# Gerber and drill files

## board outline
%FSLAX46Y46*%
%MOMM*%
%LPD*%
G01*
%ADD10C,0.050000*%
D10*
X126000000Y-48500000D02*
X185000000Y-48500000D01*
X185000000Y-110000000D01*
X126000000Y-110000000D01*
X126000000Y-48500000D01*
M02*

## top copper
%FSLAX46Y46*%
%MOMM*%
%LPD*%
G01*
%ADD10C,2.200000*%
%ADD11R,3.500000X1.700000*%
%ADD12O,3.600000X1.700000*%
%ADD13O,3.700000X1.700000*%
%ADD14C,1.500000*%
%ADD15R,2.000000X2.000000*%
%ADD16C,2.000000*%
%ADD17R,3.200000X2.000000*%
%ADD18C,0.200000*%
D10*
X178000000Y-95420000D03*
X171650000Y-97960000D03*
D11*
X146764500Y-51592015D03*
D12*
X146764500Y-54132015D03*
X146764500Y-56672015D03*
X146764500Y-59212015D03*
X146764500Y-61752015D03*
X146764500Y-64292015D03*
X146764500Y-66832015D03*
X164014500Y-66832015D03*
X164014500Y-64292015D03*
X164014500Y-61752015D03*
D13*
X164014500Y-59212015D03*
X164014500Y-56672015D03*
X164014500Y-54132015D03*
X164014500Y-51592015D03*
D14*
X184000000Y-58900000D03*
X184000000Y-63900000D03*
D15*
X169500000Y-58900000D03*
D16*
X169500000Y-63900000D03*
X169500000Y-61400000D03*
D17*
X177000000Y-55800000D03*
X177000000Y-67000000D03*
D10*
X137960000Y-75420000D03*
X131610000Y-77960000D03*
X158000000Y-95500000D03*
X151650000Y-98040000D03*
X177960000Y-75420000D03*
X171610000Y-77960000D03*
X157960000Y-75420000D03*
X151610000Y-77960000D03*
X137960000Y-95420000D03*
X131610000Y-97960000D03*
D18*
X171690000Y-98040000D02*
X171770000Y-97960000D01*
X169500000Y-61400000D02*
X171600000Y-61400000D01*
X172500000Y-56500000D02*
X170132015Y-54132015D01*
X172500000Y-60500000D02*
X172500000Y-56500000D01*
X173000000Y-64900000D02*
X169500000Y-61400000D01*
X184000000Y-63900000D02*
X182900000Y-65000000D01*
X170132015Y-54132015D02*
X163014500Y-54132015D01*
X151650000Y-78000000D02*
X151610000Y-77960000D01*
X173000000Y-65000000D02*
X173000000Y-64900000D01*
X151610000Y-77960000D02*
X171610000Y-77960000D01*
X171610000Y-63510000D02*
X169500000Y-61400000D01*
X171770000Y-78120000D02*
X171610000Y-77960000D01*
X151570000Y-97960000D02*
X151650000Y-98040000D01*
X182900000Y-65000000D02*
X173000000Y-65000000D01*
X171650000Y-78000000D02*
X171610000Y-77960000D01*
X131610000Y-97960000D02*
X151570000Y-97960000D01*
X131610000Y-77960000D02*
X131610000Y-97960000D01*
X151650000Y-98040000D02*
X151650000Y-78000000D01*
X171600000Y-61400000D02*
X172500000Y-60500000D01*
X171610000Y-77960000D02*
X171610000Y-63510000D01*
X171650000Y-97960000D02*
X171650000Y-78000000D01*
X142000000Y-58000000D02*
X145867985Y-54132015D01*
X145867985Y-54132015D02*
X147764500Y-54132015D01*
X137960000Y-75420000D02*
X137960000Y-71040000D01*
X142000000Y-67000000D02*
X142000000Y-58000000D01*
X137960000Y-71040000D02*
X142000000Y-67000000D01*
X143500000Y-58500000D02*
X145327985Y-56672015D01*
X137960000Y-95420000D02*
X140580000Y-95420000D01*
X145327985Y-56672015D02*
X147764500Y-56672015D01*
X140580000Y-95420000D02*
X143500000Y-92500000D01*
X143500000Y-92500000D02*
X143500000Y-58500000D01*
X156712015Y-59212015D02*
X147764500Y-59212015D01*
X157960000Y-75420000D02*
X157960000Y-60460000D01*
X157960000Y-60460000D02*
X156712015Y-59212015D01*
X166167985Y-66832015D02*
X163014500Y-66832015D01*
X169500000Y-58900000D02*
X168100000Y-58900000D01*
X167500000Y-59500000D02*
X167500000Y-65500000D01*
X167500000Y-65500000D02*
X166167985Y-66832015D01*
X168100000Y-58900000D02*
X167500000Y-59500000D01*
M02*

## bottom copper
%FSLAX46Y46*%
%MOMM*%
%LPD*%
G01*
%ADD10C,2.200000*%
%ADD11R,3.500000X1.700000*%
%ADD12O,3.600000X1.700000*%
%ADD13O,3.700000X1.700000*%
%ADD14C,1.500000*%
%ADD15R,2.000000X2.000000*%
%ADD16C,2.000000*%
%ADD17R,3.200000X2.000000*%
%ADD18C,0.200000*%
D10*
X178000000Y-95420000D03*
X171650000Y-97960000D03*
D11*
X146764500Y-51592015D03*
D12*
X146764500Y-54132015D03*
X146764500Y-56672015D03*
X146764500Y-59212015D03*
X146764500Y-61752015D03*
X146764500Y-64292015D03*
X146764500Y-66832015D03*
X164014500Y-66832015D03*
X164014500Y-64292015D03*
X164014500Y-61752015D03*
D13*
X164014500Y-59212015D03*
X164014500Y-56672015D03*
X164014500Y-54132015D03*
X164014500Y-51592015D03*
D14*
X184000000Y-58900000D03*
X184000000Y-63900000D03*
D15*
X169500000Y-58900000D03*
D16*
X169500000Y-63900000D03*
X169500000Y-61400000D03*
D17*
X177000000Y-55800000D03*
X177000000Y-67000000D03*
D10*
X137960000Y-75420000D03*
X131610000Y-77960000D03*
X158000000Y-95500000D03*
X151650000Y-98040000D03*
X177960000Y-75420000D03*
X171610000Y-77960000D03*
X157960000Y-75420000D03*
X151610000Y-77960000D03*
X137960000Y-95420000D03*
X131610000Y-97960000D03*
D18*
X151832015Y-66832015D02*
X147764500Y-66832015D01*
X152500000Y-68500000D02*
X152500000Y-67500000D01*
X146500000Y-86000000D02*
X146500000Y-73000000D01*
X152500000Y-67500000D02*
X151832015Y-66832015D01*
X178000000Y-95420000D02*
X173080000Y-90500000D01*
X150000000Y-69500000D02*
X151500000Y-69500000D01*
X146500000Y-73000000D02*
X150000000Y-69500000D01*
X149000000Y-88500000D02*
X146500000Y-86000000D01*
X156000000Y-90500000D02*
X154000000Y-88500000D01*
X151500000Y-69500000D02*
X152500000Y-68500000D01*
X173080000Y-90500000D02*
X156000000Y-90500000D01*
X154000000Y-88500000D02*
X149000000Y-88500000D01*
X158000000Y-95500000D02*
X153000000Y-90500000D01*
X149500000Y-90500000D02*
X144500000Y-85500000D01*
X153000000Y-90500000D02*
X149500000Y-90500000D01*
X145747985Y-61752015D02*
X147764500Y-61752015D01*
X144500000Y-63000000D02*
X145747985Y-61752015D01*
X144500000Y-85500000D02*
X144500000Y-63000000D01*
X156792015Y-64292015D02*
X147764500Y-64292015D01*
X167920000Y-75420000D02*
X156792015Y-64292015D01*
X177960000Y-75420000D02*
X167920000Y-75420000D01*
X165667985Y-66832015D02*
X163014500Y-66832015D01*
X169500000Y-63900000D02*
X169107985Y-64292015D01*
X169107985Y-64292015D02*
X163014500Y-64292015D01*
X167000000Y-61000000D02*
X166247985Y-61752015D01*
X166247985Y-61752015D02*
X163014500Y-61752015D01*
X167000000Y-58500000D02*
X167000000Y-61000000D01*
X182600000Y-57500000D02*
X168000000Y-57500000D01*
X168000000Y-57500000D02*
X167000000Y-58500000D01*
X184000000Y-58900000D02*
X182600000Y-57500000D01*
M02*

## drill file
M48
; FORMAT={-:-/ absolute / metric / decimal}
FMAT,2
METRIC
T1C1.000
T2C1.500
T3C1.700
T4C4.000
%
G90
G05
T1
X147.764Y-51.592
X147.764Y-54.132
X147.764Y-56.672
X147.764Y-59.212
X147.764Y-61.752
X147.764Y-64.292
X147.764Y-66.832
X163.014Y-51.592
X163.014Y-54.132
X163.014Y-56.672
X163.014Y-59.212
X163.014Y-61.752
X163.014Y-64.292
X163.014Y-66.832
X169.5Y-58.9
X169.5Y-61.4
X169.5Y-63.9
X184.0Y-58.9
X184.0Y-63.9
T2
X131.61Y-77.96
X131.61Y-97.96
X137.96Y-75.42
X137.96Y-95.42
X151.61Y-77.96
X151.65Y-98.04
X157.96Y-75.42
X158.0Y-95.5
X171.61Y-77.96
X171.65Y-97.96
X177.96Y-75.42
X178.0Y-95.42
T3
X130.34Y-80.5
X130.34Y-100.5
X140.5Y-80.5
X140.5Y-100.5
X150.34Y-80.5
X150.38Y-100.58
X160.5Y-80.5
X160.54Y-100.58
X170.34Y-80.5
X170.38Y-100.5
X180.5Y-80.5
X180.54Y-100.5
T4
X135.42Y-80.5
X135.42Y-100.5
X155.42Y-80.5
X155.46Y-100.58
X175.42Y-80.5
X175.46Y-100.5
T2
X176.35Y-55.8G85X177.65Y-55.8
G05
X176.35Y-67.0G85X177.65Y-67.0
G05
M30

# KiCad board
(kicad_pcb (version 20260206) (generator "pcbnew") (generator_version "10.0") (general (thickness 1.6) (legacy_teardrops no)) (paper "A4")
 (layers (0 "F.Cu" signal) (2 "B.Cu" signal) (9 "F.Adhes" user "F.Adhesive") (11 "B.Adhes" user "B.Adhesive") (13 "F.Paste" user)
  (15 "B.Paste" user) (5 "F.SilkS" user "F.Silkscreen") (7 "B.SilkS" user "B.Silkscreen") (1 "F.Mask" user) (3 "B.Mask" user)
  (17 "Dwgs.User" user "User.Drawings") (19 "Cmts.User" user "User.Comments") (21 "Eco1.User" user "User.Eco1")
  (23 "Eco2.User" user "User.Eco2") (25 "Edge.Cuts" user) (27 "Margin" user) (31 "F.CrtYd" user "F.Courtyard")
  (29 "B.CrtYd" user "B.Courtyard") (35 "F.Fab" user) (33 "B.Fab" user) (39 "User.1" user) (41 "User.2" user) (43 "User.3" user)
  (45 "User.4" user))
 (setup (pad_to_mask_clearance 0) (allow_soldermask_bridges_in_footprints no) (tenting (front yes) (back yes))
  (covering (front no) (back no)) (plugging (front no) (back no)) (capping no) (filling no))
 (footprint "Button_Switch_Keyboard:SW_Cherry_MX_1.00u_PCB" (layer "F.Cu") (at 178 95.42)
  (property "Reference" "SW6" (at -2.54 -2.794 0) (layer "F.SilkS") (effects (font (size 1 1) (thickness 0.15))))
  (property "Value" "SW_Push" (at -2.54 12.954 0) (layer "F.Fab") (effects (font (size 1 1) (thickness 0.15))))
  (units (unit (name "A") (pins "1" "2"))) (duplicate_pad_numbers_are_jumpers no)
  (pad "" np_thru_hole circle (at -7.62 5.08) (size 1.7 1.7) (drill 1.7) (layers "*.Cu" "*.Mask"))
  (pad "" np_thru_hole circle (at -2.54 5.08) (size 4 4) (drill 4) (layers "*.Cu" "*.Mask"))
  (pad "" np_thru_hole circle (at 2.54 5.08) (size 1.7 1.7) (drill 1.7) (layers "*.Cu" "*.Mask"))
  (pad "1" thru_hole circle (at 0 0) (size 2.2 2.2) (drill 1.5) (layers "*.Cu" "*.Mask") (remove_unused_layers no)
   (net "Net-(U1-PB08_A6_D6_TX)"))
  (pad "2" thru_hole circle (at -6.35 2.54) (size 2.2 2.2) (drill 1.5) (layers "*.Cu" "*.Mask") (remove_unused_layers no) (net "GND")))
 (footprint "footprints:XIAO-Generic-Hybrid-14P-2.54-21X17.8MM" (layer "F.Cu") (at 155.3895 59.212015)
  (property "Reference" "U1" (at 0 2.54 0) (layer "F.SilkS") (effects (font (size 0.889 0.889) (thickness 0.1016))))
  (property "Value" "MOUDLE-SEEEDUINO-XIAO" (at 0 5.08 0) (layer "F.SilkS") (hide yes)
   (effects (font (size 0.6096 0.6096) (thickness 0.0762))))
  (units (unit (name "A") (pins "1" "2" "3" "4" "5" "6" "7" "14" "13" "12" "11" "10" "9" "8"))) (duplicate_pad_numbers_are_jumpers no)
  (pad "1" thru_hole rect (at -7.625 -7.62) (size 3.5 1.7) (drill 1 (offset -1 0)) (layers "*.Cu" "*.Mask") (remove_unused_layers no)
   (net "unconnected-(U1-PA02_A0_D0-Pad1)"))
  (pad "2" thru_hole oval (at -7.625 -5.08) (size 3.6 1.7) (drill 1 (offset -1 0)) (layers "*.Cu" "*.Mask") (remove_unused_layers no)
   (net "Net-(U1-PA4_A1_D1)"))
  (pad "3" thru_hole oval (at -7.625 -2.54) (size 3.6 1.7) (drill 1 (offset -1 0)) (layers "*.Cu" "*.Mask") (remove_unused_layers no)
   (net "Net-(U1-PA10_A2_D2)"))
  (pad "4" thru_hole oval (at -7.625 0) (size 3.6 1.7) (drill 1 (offset -1 0)) (layers "*.Cu" "*.Mask") (remove_unused_layers no)
   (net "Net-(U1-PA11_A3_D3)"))
  (pad "5" thru_hole oval (at -7.625 2.54) (size 3.6 1.7) (drill 1 (offset -1 0)) (layers "*.Cu" "*.Mask") (remove_unused_layers no)
   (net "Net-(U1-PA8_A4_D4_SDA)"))
  (pad "6" thru_hole oval (at -7.625 5.08 180) (size 3.6 1.7) (drill 1 (offset 1 0)) (layers "*.Cu" "*.Mask") (remove_unused_layers no)
   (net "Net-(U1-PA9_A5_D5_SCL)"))
  (pad "7" thru_hole oval (at -7.625 7.62) (size 3.6 1.7) (drill 1 (offset -1 0)) (layers "*.Cu" "*.Mask") (remove_unused_layers no)
   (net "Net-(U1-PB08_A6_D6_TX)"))
  (pad "8" thru_hole oval (at 7.625 7.62) (size 3.6 1.7) (drill 1 (offset 1 0)) (layers "*.Cu" "*.Mask") (remove_unused_layers no)
   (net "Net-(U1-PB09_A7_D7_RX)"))
  (pad "9" thru_hole oval (at 7.625 5.08) (size 3.6 1.7) (drill 1 (offset 1 0)) (layers "*.Cu" "*.Mask") (remove_unused_layers no)
   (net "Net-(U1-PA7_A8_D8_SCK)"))
  (pad "10" thru_hole oval (at 7.625 2.54) (size 3.6 1.7) (drill 1 (offset 1 0)) (layers "*.Cu" "*.Mask") (remove_unused_layers no)
   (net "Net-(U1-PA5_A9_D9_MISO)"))
  (pad "11" thru_hole oval (at 7.625 0) (size 3.7 1.7) (drill 1 (offset 1 0)) (layers "*.Cu" "*.Mask") (remove_unused_layers no)
   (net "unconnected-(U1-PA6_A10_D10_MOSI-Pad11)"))
  (pad "12" thru_hole oval (at 7.625 -2.54) (size 3.7 1.7) (drill 1 (offset 1 0)) (layers "*.Cu" "*.Mask") (remove_unused_layers no)
   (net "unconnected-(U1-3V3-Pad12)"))
  (pad "13" thru_hole oval (at 7.625 -5.08) (size 3.7 1.7) (drill 1 (offset 1 0)) (layers "*.Cu" "*.Mask") (remove_unused_layers no)
   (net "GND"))
  (pad "14" thru_hole oval (at 7.625 -7.62) (size 3.7 1.7) (drill 1 (offset 1 0)) (layers "*.Cu" "*.Mask") (remove_unused_layers no)
   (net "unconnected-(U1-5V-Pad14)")))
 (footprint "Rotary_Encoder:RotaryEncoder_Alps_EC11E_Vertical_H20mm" (layer "F.Cu") (at 169.5 58.9)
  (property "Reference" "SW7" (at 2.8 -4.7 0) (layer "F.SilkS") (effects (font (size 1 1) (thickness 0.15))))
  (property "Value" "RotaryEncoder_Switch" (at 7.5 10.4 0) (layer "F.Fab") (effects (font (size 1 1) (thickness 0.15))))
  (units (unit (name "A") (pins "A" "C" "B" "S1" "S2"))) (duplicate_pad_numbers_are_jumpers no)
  (pad "" thru_hole circle (at 14.5 0) (size 1.5 1.5) (drill 1) (layers "*.Cu" "*.Mask") (remove_unused_layers no)
   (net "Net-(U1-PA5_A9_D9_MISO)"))
  (pad "" thru_hole circle (at 14.5 5) (size 1.5 1.5) (drill 1) (layers "*.Cu" "*.Mask") (remove_unused_layers no) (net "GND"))
  (pad "A" thru_hole rect (at 0 0) (size 2 2) (drill 1) (layers "*.Cu" "*.Mask") (remove_unused_layers no) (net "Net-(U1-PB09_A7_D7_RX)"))
  (pad "B" thru_hole circle (at 0 5) (size 2 2) (drill 1) (layers "*.Cu" "*.Mask") (remove_unused_layers no) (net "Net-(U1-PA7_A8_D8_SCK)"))
  (pad "C" thru_hole circle (at 0 2.5) (size 2 2) (drill 1) (layers "*.Cu" "*.Mask") (remove_unused_layers no) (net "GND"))
  (pad "MP" thru_hole rect (at 7.5 -3.1) (size 3.2 2) (drill oval 2.8 1.5) (layers "*.Cu" "*.Mask") (remove_unused_layers no))
  (pad "MP" thru_hole rect (at 7.5 8.1) (size 3.2 2) (drill oval 2.8 1.5) (layers "*.Cu" "*.Mask") (remove_unused_layers no)))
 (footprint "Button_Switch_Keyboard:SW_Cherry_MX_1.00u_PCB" (layer "F.Cu") (at 137.96 75.42)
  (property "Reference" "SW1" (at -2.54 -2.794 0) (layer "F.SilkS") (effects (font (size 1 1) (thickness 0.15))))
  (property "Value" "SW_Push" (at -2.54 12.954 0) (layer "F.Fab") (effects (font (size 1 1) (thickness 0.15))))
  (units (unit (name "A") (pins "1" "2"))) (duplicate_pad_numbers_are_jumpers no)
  (pad "" np_thru_hole circle (at -7.62 5.08) (size 1.7 1.7) (drill 1.7) (layers "*.Cu" "*.Mask"))
  (pad "" np_thru_hole circle (at -2.54 5.08) (size 4 4) (drill 4) (layers "*.Cu" "*.Mask"))
  (pad "" np_thru_hole circle (at 2.54 5.08) (size 1.7 1.7) (drill 1.7) (layers "*.Cu" "*.Mask"))
  (pad "1" thru_hole circle (at 0 0) (size 2.2 2.2) (drill 1.5) (layers "*.Cu" "*.Mask") (remove_unused_layers no)
   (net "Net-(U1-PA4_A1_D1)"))
  (pad "2" thru_hole circle (at -6.35 2.54) (size 2.2 2.2) (drill 1.5) (layers "*.Cu" "*.Mask") (remove_unused_layers no) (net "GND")))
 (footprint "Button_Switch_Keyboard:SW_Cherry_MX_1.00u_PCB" (layer "F.Cu") (at 158 95.5)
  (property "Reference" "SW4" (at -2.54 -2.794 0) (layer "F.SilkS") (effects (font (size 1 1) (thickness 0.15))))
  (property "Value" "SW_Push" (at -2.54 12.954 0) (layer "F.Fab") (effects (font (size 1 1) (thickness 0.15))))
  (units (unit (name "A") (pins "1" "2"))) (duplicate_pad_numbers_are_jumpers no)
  (pad "" np_thru_hole circle (at -7.62 5.08) (size 1.7 1.7) (drill 1.7) (layers "*.Cu" "*.Mask"))
  (pad "" np_thru_hole circle (at -2.54 5.08) (size 4 4) (drill 4) (layers "*.Cu" "*.Mask"))
  (pad "" np_thru_hole circle (at 2.54 5.08) (size 1.7 1.7) (drill 1.7) (layers "*.Cu" "*.Mask"))
  (pad "1" thru_hole circle (at 0 0) (size 2.2 2.2) (drill 1.5) (layers "*.Cu" "*.Mask") (remove_unused_layers no)
   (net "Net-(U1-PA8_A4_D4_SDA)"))
  (pad "2" thru_hole circle (at -6.35 2.54) (size 2.2 2.2) (drill 1.5) (layers "*.Cu" "*.Mask") (remove_unused_layers no) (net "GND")))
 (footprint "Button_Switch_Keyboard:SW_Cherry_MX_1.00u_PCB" (layer "F.Cu") (at 177.96 75.42)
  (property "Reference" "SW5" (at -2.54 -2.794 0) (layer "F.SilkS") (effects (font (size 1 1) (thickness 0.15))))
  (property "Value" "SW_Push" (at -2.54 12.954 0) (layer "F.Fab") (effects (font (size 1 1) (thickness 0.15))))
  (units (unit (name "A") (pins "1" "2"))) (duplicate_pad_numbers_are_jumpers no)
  (pad "" np_thru_hole circle (at -7.62 5.08) (size 1.7 1.7) (drill 1.7) (layers "*.Cu" "*.Mask"))
  (pad "" np_thru_hole circle (at -2.54 5.08) (size 4 4) (drill 4) (layers "*.Cu" "*.Mask"))
  (pad "" np_thru_hole circle (at 2.54 5.08) (size 1.7 1.7) (drill 1.7) (layers "*.Cu" "*.Mask"))
  (pad "1" thru_hole circle (at 0 0) (size 2.2 2.2) (drill 1.5) (layers "*.Cu" "*.Mask") (remove_unused_layers no)
   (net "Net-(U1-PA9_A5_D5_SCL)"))
  (pad "2" thru_hole circle (at -6.35 2.54) (size 2.2 2.2) (drill 1.5) (layers "*.Cu" "*.Mask") (remove_unused_layers no) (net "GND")))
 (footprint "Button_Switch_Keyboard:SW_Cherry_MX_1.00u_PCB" (layer "F.Cu") (at 157.96 75.42)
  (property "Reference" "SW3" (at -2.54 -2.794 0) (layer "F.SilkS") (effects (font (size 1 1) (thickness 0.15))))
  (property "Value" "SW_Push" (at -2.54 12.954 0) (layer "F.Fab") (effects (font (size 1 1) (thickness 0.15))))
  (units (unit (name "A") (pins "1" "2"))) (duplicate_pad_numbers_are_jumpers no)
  (pad "" np_thru_hole circle (at -7.62 5.08) (size 1.7 1.7) (drill 1.7) (layers "*.Cu" "*.Mask"))
  (pad "" np_thru_hole circle (at -2.54 5.08) (size 4 4) (drill 4) (layers "*.Cu" "*.Mask"))
  (pad "" np_thru_hole circle (at 2.54 5.08) (size 1.7 1.7) (drill 1.7) (layers "*.Cu" "*.Mask"))
  (pad "1" thru_hole circle (at 0 0) (size 2.2 2.2) (drill 1.5) (layers "*.Cu" "*.Mask") (remove_unused_layers no)
   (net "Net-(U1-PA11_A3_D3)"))
  (pad "2" thru_hole circle (at -6.35 2.54) (size 2.2 2.2) (drill 1.5) (layers "*.Cu" "*.Mask") (remove_unused_layers no) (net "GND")))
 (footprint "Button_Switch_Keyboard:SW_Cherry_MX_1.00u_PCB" (layer "F.Cu") (at 137.96 95.42)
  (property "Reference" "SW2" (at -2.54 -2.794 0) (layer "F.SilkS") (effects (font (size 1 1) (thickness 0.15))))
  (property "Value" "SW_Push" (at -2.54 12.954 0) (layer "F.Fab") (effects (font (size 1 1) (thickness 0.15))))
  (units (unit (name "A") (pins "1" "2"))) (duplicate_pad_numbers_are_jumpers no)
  (pad "" np_thru_hole circle (at -7.62 5.08) (size 1.7 1.7) (drill 1.7) (layers "*.Cu" "*.Mask"))
  (pad "" np_thru_hole circle (at -2.54 5.08) (size 4 4) (drill 4) (layers "*.Cu" "*.Mask"))
  (pad "" np_thru_hole circle (at 2.54 5.08) (size 1.7 1.7) (drill 1.7) (layers "*.Cu" "*.Mask"))
  (pad "1" thru_hole circle (at 0 0) (size 2.2 2.2) (drill 1.5) (layers "*.Cu" "*.Mask") (remove_unused_layers no)
   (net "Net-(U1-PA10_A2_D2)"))
  (pad "2" thru_hole circle (at -6.35 2.54) (size 2.2 2.2) (drill 1.5) (layers "*.Cu" "*.Mask") (remove_unused_layers no) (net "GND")))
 (gr_rect (start 126 48.5) (end 185 110) (stroke (width 0.05) (type default)) (fill no) (layer "Edge.Cuts"))
 (segment (start 151.832015 66.832015) (end 147.7645 66.832015) (width 0.2) (layer "B.Cu") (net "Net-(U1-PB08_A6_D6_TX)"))
 (segment (start 152.5 68.5) (end 152.5 67.5) (width 0.2) (layer "B.Cu") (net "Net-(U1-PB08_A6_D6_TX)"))
 (segment (start 146.5 86) (end 146.5 73) (width 0.2) (layer "B.Cu") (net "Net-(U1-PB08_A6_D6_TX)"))
 (segment (start 152.5 67.5) (end 151.832015 66.832015) (width 0.2) (layer "B.Cu") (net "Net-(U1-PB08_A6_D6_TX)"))
 (segment (start 178 95.42) (end 173.08 90.5) (width 0.2) (layer "B.Cu") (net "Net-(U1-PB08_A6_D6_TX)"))
 (segment (start 150 69.5) (end 151.5 69.5) (width 0.2) (layer "B.Cu") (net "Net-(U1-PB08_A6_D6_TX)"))
 (segment (start 146.5 73) (end 150 69.5) (width 0.2) (layer "B.Cu") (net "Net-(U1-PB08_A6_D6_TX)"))
 (segment (start 149 88.5) (end 146.5 86) (width 0.2) (layer "B.Cu") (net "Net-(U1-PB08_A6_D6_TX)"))
 (segment (start 156 90.5) (end 154 88.5) (width 0.2) (layer "B.Cu") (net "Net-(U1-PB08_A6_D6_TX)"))
 (segment (start 151.5 69.5) (end 152.5 68.5) (width 0.2) (layer "B.Cu") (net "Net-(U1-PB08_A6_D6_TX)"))
 (segment (start 173.08 90.5) (end 156 90.5) (width 0.2) (layer "B.Cu") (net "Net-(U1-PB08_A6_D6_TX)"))
 (segment (start 154 88.5) (end 149 88.5) (width 0.2) (layer "B.Cu") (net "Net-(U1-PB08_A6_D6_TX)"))
 (segment (start 171.69 98.04) (end 171.77 97.96) (width 0.2) (layer "F.Cu") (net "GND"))
 (segment (start 169.5 61.4) (end 171.6 61.4) (width 0.2) (layer "F.Cu") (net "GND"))
 (segment (start 172.5 56.5) (end 170.132015 54.132015) (width 0.2) (layer "F.Cu") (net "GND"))
 (segment (start 172.5 60.5) (end 172.5 56.5) (width 0.2) (layer "F.Cu") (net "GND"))
 (segment (start 173 64.9) (end 169.5 61.4) (width 0.2) (layer "F.Cu") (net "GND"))
 (segment (start 184 63.9) (end 182.9 65) (width 0.2) (layer "F.Cu") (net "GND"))
 (segment (start 170.132015 54.132015) (end 163.0145 54.132015) (width 0.2) (layer "F.Cu") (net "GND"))
 (segment (start 151.65 78) (end 151.61 77.96) (width 0.2) (layer "F.Cu") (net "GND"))
 (segment (start 173 65) (end 173 64.9) (width 0.2) (layer "F.Cu") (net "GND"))
 (segment (start 151.61 77.96) (end 171.61 77.96) (width 0.2) (layer "F.Cu") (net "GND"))
 (segment (start 171.61 63.51) (end 169.5 61.4) (width 0.2) (layer "F.Cu") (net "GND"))
 (segment (start 171.77 78.12) (end 171.61 77.96) (width 0.2) (layer "F.Cu") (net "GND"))
 (segment (start 151.57 97.96) (end 151.65 98.04) (width 0.2) (layer "F.Cu") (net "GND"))
 (segment (start 182.9 65) (end 173 65) (width 0.2) (layer "F.Cu") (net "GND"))
 (segment (start 171.65 78) (end 171.61 77.96) (width 0.2) (layer "F.Cu") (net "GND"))
 (segment (start 131.61 97.96) (end 151.57 97.96) (width 0.2) (layer "F.Cu") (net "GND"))
 (segment (start 131.61 77.96) (end 131.61 97.96) (width 0.2) (layer "F.Cu") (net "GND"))
 (segment (start 151.65 98.04) (end 151.65 78) (width 0.2) (layer "F.Cu") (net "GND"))
 (segment (start 171.6 61.4) (end 172.5 60.5) (width 0.2) (layer "F.Cu") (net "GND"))
 (segment (start 171.61 77.96) (end 171.61 63.51) (width 0.2) (layer "F.Cu") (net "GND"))
 (segment (start 171.65 97.96) (end 171.65 78) (width 0.2) (layer "F.Cu") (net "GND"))
 (segment (start 142 58) (end 145.867985 54.132015) (width 0.2) (layer "F.Cu") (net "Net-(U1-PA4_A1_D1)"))
 (segment (start 145.867985 54.132015) (end 147.7645 54.132015) (width 0.2) (layer "F.Cu") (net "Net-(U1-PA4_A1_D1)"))
 (segment (start 137.96 75.42) (end 137.96 71.04) (width 0.2) (layer "F.Cu") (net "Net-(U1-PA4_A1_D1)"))
 (segment (start 142 67) (end 142 58) (width 0.2) (layer "F.Cu") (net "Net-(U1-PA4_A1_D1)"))
 (segment (start 137.96 71.04) (end 142 67) (width 0.2) (layer "F.Cu") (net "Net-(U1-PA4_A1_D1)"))
 (segment (start 143.5 58.5) (end 145.327985 56.672015) (width 0.2) (layer "F.Cu") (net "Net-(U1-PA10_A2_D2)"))
 (segment (start 137.96 95.42) (end 140.58 95.42) (width 0.2) (layer "F.Cu") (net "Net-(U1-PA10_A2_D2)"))
 (segment (start 145.327985 56.672015) (end 147.7645 56.672015) (width 0.2) (layer "F.Cu") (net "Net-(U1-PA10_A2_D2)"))
 (segment (start 140.58 95.42) (end 143.5 92.5) (width 0.2) (layer "F.Cu") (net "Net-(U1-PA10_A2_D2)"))
 (segment (start 143.5 92.5) (end 143.5 58.5) (width 0.2) (layer "F.Cu") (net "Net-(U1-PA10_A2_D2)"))
 (segment (start 156.712015 59.212015) (end 147.7645 59.212015) (width 0.2) (layer "F.Cu") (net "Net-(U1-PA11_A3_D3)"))
 (segment (start 157.96 75.42) (end 157.96 60.46) (width 0.2) (layer "F.Cu") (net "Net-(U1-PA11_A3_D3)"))
 (segment (start 157.96 60.46) (end 156.712015 59.212015) (width 0.2) (layer "F.Cu") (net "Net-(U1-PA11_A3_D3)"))
 (segment (start 158 95.5) (end 153 90.5) (width 0.2) (layer "B.Cu") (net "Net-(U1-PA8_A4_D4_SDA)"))
 (segment (start 149.5 90.5) (end 144.5 85.5) (width 0.2) (layer "B.Cu") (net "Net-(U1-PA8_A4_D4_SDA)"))
 (segment (start 153 90.5) (end 149.5 90.5) (width 0.2) (layer "B.Cu") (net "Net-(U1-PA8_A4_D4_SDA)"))
 (segment (start 145.747985 61.752015) (end 147.7645 61.752015) (width 0.2) (layer "B.Cu") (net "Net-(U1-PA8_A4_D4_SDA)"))
 (segment (start 144.5 63) (end 145.747985 61.752015) (width 0.2) (layer "B.Cu") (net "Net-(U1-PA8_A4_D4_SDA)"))
 (segment (start 144.5 85.5) (end 144.5 63) (width 0.2) (layer "B.Cu") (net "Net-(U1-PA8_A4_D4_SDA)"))
 (segment (start 156.792015 64.292015) (end 147.7645 64.292015) (width 0.2) (layer "B.Cu") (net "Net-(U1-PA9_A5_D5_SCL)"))
 (segment (start 167.92 75.42) (end 156.792015 64.292015) (width 0.2) (layer "B.Cu") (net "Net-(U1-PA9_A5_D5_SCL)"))
 (segment (start 177.96 75.42) (end 167.92 75.42) (width 0.2) (layer "B.Cu") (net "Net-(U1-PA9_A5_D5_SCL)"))
 (segment (start 166.167985 66.832015) (end 163.0145 66.832015) (width 0.2) (layer "F.Cu") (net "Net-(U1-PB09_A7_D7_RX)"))
 (segment (start 169.5 58.9) (end 168.1 58.9) (width 0.2) (layer "F.Cu") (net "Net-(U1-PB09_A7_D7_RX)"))
 (segment (start 167.5 59.5) (end 167.5 65.5) (width 0.2) (layer "F.Cu") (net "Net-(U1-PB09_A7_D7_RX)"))
 (segment (start 167.5 65.5) (end 166.167985 66.832015) (width 0.2) (layer "F.Cu") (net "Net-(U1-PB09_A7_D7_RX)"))
 (segment (start 168.1 58.9) (end 167.5 59.5) (width 0.2) (layer "F.Cu") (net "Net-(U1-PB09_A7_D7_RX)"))
 (segment (start 165.667985 66.832015) (end 163.0145 66.832015) (width 0.2) (layer "B.Cu") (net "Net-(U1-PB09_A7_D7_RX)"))
 (segment (start 169.5 63.9) (end 169.107985 64.292015) (width 0.2) (layer "B.Cu") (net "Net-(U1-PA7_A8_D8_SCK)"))
 (segment (start 169.107985 64.292015) (end 163.0145 64.292015) (width 0.2) (layer "B.Cu") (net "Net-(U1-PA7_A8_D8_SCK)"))
 (segment (start 167 61) (end 166.247985 61.752015) (width 0.2) (layer "B.Cu") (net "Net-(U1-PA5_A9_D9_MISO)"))
 (segment (start 166.247985 61.752015) (end 163.0145 61.752015) (width 0.2) (layer "B.Cu") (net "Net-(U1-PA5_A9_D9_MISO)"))
 (segment (start 167 58.5) (end 167 61) (width 0.2) (layer "B.Cu") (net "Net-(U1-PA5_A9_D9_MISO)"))
 (segment (start 182.6 57.5) (end 168 57.5) (width 0.2) (layer "B.Cu") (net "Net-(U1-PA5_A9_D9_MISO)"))
 (segment (start 168 57.5) (end 167 58.5) (width 0.2) (layer "B.Cu") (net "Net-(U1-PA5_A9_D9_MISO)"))
 (segment (start 184 58.9) (end 182.6 57.5) (width 0.2) (layer "B.Cu") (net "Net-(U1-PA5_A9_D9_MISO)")))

